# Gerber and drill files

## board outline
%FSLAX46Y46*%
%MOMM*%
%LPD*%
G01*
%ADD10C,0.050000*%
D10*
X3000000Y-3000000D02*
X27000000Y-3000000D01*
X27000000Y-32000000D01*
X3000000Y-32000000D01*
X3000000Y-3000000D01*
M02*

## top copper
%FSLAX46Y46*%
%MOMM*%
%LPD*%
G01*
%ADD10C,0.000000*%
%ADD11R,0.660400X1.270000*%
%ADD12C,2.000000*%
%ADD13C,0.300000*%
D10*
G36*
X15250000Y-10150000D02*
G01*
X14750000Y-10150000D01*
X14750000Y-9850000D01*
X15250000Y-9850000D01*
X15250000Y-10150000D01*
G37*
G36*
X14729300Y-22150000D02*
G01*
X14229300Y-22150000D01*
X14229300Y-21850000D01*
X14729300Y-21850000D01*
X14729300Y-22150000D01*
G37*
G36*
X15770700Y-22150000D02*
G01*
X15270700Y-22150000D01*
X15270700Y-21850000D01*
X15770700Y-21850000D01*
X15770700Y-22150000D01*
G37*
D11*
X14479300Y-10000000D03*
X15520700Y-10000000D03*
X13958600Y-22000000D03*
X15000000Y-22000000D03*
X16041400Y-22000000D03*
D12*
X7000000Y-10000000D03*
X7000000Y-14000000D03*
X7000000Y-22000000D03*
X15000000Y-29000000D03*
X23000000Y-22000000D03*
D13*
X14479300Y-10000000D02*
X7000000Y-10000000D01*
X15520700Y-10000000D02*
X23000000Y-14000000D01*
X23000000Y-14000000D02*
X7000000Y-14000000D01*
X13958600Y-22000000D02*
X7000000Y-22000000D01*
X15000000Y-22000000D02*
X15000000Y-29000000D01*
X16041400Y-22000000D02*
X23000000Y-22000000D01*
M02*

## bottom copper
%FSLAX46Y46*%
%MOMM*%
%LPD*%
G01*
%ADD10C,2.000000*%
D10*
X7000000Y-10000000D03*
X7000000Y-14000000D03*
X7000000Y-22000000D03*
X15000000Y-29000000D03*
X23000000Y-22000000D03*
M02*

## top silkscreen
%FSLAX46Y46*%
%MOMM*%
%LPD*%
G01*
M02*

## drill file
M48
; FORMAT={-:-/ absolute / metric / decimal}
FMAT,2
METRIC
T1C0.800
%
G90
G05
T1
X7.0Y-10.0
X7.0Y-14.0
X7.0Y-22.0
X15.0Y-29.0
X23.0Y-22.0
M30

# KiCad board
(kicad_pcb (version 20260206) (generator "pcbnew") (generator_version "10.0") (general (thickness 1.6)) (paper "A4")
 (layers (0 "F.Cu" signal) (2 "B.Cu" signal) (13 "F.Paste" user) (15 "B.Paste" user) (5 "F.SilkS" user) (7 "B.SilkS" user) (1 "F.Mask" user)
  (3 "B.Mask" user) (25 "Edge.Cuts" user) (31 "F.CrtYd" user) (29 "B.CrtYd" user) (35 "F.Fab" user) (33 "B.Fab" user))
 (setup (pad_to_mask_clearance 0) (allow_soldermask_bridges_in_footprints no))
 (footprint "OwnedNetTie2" (layer "F.Cu") (at 15 10)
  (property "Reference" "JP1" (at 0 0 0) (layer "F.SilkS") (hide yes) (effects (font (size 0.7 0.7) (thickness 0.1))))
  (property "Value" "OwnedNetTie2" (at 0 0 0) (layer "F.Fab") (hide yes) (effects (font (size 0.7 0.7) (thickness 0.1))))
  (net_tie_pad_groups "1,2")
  (fp_poly (pts (xy -0.25 -0.15) (xy 0.25 -0.15) (xy 0.25 0.15) (xy -0.25 0.15)) (stroke (width 0) (type solid)) (fill yes) (layer "F.Cu"))
  (pad "1" smd rect (at -0.5207 0) (size 0.6604 1.27) (layers "F.Cu" "F.Mask") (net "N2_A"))
  (pad "2" smd rect (at 0.5207 0) (size 0.6604 1.27) (layers "F.Cu" "F.Mask") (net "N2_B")))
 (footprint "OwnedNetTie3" (layer "F.Cu") (at 15 22)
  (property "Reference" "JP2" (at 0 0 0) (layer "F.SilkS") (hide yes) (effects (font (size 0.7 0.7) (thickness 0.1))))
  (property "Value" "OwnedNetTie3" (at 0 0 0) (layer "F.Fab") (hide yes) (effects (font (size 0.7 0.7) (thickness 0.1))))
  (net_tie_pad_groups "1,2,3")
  (fp_poly
   (pts (xy -0.7707 -0.15) (xy -0.2707 -0.15) (xy -0.2707 0.15) (xy -0.7707 0.15)) (stroke (width 0) (type solid)) (fill yes) (layer "F.Cu"))
  (fp_poly
   (pts (xy 0.2707 -0.15) (xy 0.7707 -0.15) (xy 0.7707 0.15) (xy 0.2707 0.15)) (stroke (width 0) (type solid)) (fill yes) (layer "F.Cu"))
  (pad "1" smd rect (at -1.0414 0) (size 0.6604 1.27) (layers "F.Cu" "F.Mask") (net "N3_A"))
  (pad "2" smd rect (at 0 0) (size 0.6604 1.27) (layers "F.Cu" "F.Mask") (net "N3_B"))
  (pad "3" smd rect (at 1.0414 0) (size 0.6604 1.27) (layers "F.Cu" "F.Mask") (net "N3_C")))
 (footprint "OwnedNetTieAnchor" (layer "F.Cu") (at 7 10)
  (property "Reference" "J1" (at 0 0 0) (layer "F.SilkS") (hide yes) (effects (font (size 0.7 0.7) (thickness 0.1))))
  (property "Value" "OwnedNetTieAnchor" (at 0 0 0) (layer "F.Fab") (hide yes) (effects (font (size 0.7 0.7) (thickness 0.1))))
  (pad "1" thru_hole circle (at 0 0) (size 2 2) (drill 0.8) (layers "*.Cu" "*.Mask") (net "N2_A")))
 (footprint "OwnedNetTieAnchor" (layer "F.Cu") (at 7 14)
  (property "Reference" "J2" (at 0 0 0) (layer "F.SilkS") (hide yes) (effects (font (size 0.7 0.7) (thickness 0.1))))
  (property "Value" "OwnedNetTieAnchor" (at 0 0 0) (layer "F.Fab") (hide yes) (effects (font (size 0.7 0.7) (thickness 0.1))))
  (pad "1" thru_hole circle (at 0 0) (size 2 2) (drill 0.8) (layers "*.Cu" "*.Mask") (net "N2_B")))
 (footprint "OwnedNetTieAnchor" (layer "F.Cu") (at 7 22)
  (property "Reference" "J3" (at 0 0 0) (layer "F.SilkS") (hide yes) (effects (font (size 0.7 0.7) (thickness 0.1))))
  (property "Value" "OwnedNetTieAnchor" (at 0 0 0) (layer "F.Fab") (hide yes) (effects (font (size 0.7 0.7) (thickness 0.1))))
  (pad "1" thru_hole circle (at 0 0) (size 2 2) (drill 0.8) (layers "*.Cu" "*.Mask") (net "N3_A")))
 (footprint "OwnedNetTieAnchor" (layer "F.Cu") (at 15 29)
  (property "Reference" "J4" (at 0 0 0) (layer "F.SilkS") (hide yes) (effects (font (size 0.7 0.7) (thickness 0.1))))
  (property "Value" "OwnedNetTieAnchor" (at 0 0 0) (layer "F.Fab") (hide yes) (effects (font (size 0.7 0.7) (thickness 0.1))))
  (pad "1" thru_hole circle (at 0 0) (size 2 2) (drill 0.8) (layers "*.Cu" "*.Mask") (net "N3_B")))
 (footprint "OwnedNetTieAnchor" (layer "F.Cu") (at 23 22)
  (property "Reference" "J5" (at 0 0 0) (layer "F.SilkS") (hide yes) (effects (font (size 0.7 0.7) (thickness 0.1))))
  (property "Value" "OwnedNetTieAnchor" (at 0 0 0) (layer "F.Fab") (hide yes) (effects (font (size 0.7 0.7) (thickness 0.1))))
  (pad "1" thru_hole circle (at 0 0) (size 2 2) (drill 0.8) (layers "*.Cu" "*.Mask") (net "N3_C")))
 (segment (start 14.4793 10) (end 7 10) (width 0.3) (layer "F.Cu") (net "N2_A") (locked yes))
 (segment (start 15.5207 10) (end 23 14) (width 0.3) (layer "F.Cu") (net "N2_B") (locked yes))
 (segment (start 23 14) (end 7 14) (width 0.3) (layer "F.Cu") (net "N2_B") (locked yes))
 (segment (start 13.9586 22) (end 7 22) (width 0.3) (layer "F.Cu") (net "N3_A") (locked yes))
 (segment (start 15 22) (end 15 29) (width 0.3) (layer "F.Cu") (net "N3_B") (locked yes))
 (segment (start 16.0414 22) (end 23 22) (width 0.3) (layer "F.Cu") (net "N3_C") (locked yes))
 (gr_rect (start 3 3) (end 27 32) (stroke (width 0.05) (type default)) (fill none) (layer "Edge.Cuts")))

